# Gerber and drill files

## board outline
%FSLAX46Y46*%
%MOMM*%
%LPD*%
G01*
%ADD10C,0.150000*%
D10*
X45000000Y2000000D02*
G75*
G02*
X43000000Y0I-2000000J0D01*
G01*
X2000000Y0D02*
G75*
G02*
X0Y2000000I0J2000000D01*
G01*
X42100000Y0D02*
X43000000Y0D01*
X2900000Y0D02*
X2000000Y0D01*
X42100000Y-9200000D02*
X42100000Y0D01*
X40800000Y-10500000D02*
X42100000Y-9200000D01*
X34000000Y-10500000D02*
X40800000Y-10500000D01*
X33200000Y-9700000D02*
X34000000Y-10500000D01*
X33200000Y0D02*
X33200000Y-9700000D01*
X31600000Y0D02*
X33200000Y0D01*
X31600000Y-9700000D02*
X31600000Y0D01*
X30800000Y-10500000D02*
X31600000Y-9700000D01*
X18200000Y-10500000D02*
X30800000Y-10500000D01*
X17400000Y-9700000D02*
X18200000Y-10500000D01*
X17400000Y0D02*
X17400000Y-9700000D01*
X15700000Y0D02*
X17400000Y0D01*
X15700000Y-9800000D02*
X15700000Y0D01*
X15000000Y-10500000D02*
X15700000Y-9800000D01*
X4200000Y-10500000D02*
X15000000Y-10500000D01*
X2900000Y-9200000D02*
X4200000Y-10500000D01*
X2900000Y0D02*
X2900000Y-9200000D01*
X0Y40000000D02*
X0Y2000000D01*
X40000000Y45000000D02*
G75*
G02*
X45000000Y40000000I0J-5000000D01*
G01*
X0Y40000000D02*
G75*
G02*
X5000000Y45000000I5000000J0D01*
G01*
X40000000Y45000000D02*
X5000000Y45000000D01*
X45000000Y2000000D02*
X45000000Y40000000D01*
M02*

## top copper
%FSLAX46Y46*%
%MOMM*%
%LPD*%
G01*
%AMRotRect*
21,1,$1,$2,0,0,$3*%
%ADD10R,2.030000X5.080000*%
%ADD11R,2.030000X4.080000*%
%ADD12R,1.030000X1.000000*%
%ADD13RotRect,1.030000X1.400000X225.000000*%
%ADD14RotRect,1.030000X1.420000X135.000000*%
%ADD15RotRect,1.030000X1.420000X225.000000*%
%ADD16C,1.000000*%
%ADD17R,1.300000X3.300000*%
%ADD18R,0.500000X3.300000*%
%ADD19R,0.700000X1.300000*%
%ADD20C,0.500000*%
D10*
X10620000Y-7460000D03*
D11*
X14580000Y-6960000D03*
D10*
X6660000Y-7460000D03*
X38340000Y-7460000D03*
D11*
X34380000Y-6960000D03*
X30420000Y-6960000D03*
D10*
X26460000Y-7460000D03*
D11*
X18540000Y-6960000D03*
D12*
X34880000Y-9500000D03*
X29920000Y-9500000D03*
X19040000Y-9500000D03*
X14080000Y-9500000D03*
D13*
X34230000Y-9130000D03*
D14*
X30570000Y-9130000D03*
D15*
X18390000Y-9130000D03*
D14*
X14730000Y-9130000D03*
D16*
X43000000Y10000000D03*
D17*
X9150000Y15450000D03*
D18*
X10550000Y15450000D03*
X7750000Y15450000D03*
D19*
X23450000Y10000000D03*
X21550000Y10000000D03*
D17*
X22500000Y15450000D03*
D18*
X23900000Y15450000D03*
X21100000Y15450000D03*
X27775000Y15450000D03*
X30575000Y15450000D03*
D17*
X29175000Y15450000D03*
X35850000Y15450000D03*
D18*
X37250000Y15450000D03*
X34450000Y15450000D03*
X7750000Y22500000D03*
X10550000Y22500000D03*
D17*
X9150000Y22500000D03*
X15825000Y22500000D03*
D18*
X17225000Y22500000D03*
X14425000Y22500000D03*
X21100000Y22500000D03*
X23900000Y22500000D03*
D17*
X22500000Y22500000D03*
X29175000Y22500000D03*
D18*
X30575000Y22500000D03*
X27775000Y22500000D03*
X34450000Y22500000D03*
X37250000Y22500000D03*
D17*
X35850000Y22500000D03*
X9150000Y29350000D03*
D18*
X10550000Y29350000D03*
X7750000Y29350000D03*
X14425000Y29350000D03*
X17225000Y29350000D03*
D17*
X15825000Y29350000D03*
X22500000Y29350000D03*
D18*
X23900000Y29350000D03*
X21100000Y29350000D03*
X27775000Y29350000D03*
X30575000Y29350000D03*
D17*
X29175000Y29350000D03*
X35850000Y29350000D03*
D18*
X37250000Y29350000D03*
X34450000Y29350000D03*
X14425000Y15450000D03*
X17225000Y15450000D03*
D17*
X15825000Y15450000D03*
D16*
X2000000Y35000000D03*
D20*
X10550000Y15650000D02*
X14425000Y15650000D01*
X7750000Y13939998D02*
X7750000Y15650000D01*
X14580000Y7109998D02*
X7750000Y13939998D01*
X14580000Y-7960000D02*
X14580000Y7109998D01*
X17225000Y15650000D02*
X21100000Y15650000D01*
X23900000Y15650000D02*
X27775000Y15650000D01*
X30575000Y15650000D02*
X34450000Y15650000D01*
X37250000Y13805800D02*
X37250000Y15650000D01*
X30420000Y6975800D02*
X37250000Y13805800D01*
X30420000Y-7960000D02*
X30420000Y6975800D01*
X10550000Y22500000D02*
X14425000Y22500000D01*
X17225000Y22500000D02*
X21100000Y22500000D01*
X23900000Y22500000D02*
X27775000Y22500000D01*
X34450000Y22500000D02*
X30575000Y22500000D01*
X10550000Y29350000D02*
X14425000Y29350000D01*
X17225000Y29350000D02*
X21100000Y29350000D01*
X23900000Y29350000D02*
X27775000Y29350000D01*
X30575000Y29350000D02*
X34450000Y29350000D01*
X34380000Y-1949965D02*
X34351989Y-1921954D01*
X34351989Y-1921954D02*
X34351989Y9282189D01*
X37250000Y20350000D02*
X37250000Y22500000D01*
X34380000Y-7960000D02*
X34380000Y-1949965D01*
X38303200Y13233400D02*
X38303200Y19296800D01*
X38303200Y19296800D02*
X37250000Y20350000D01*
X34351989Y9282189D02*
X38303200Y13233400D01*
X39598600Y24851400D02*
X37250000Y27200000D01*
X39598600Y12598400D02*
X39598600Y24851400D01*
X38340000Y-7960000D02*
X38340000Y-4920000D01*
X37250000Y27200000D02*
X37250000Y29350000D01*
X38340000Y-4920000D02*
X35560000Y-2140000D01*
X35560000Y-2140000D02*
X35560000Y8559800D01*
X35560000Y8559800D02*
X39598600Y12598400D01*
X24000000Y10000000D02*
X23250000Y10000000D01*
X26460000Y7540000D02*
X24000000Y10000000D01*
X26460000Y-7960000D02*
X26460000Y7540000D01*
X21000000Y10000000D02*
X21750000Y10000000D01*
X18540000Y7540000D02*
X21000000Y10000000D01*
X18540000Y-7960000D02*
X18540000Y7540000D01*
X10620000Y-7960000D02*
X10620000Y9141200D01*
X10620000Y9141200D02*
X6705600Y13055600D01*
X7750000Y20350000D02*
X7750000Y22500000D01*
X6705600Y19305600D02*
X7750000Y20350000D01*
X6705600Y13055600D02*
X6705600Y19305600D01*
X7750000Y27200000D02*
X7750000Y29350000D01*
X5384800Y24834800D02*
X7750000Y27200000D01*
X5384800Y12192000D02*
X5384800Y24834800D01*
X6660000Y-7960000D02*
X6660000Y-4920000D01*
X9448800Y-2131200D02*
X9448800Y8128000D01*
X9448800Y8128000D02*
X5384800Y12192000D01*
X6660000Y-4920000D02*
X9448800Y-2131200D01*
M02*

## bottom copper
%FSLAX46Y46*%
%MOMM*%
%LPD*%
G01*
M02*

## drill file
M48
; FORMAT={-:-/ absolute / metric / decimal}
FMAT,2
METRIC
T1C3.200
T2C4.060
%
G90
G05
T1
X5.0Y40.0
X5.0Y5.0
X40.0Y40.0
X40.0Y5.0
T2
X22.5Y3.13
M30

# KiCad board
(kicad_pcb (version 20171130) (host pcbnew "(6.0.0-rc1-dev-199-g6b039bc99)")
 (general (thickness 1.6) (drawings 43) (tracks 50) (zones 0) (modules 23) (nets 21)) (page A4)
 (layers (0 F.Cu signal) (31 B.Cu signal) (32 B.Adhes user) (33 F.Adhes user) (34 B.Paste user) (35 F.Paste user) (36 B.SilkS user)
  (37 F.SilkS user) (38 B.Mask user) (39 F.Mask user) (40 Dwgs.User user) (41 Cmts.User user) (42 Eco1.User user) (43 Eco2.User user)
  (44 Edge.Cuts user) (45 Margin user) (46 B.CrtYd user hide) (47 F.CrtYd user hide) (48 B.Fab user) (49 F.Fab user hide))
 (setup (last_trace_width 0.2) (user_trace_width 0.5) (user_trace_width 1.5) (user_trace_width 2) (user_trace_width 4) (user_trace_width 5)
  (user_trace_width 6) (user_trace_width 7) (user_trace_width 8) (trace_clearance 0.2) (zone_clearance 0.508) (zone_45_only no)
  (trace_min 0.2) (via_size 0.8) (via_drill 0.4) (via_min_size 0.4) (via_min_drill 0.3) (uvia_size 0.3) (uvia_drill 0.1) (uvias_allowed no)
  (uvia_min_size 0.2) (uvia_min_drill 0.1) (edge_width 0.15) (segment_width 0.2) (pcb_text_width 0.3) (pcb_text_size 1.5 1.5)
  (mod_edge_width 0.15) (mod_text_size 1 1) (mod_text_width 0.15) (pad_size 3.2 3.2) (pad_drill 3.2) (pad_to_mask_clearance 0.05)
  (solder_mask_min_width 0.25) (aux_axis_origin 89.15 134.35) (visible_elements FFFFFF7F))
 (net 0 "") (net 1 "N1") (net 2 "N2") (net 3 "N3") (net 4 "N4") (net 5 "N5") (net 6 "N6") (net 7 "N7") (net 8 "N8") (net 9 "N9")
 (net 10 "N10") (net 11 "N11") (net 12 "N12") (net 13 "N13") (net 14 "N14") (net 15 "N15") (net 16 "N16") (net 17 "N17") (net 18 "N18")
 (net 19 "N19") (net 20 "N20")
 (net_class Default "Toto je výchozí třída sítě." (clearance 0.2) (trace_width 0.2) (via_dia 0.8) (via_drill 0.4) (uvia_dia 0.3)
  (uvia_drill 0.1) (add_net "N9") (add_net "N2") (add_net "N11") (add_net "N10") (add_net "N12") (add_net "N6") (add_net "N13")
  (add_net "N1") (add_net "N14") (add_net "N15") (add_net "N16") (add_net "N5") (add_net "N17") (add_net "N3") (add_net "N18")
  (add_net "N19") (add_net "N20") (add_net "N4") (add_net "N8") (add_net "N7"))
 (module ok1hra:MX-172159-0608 (layer F.Cu) (at 22.5 10.5 180)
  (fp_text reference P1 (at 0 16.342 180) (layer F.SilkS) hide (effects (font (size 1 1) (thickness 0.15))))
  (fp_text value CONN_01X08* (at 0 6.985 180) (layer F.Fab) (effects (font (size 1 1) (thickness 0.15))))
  (pad 2 smd rect (at 11.88 3.04 180) (size 2.03 5.08) (layers F.Cu F.Mask) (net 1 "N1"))
  (pad 3 smd rect (at 7.92 3.54 180) (size 2.03 4.08) (layers F.Cu F.Mask) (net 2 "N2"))
  (pad 1 smd rect (at 15.84 3.04 180) (size 2.03 5.08) (layers F.Cu F.Mask) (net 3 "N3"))
  (pad 8 smd rect (at -15.84 3.04 180) (size 2.03 5.08) (layers F.Cu F.Mask) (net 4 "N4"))
  (pad 7 smd rect (at -11.88 3.54 180) (size 2.03 4.08) (layers F.Cu F.Mask) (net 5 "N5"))
  (pad 6 smd rect (at -7.92 3.54 180) (size 2.03 4.08) (layers F.Cu F.Mask) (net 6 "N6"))
  (pad 5 smd rect (at -3.96 3.04 180) (size 2.03 5.08) (layers F.Cu F.Mask) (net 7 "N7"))
  (pad 4 smd rect (at 3.96 3.54 180) (size 2.03 4.08) (layers F.Cu F.Mask) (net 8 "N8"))
  (pad "" np_thru_hole circle (at 0 13.63 180) (size 4.06 4.06) (drill 4.06) (layers *.Cu *.Mask))
  (pad 7 smd rect (at -12.38 1 180) (size 1.03 1) (layers F.Cu F.Mask) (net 5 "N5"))
  (pad 6 smd rect (at -7.42 1 180) (size 1.03 1) (layers F.Cu F.Mask) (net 6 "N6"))
  (pad 4 smd rect (at 3.46 1 180) (size 1.03 1) (layers F.Cu F.Mask) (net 8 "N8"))
  (pad 3 smd rect (at 8.42 1 180) (size 1.03 1) (layers F.Cu F.Mask) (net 2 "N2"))
  (pad 7 smd rect (at -11.73 1.37 225) (size 1.03 1.4) (layers F.Cu F.Mask) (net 5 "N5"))
  (pad 6 smd rect (at -8.07 1.37 135) (size 1.03 1.42) (layers F.Cu F.Mask) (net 6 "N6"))
  (pad 4 smd rect (at 4.11 1.37 225) (size 1.03 1.42) (layers F.Cu F.Mask) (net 8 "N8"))
  (pad 3 smd rect (at 7.77 1.37 135) (size 1.03 1.42) (layers F.Cu F.Mask) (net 2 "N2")))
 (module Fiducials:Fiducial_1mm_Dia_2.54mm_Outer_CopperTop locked (layer F.Cu) (at 43 -10)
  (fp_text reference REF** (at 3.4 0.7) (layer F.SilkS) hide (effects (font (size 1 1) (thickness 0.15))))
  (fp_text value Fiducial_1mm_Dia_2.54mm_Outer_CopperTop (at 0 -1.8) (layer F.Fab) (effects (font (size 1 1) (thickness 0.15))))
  (pad ~ smd circle (at 0 0) (size 1 1) (layers F.Cu F.Mask) (solder_mask_margin 0.77) (clearance 0.77)))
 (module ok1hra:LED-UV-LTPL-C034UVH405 (layer F.Cu) (at 9.15 -15.45 180)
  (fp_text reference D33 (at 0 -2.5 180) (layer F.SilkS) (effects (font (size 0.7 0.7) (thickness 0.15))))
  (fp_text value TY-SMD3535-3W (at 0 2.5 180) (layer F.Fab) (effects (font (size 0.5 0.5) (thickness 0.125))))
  (pad 3 smd rect (at 0 0 180) (size 1.3 3.3) (layers F.Cu F.Paste F.Mask))
  (pad 1 smd rect (at -1.4 0 180) (size 0.5 3.3) (layers F.Cu F.Paste F.Mask) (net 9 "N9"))
  (pad 2 smd rect (at 1.4 0 180) (size 0.5 3.3) (layers F.Cu F.Paste F.Mask) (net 2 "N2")))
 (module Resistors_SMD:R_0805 (layer F.Cu) (at 22.5 -10 180)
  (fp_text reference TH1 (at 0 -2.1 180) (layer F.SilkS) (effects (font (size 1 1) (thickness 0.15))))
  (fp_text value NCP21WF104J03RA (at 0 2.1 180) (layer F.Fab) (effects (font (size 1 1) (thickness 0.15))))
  (pad 1 smd rect (at -0.95 0 180) (size 0.7 1.3) (layers F.Cu F.Paste F.Mask) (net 7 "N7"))
  (pad 2 smd rect (at 0.95 0 180) (size 0.7 1.3) (layers F.Cu F.Paste F.Mask) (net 8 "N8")))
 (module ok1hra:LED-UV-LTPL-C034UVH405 (layer F.Cu) (at 22.5 -15.45 180)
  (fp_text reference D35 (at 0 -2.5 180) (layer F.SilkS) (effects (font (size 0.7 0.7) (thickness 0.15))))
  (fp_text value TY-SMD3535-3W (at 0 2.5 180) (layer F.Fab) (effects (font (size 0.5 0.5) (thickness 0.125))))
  (pad 3 smd rect (at 0 0 180) (size 1.3 3.3) (layers F.Cu F.Paste F.Mask))
  (pad 1 smd rect (at -1.4 0 180) (size 0.5 3.3) (layers F.Cu F.Paste F.Mask) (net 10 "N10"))
  (pad 2 smd rect (at 1.4 0 180) (size 0.5 3.3) (layers F.Cu F.Paste F.Mask) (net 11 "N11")))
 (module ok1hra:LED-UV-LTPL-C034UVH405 (layer F.Cu) (at 29.175 -15.45 180)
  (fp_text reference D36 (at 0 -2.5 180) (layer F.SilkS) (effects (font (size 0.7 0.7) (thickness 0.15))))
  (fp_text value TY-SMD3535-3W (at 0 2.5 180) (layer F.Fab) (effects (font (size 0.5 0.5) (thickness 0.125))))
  (pad 2 smd rect (at 1.4 0 180) (size 0.5 3.3) (layers F.Cu F.Paste F.Mask) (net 10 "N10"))
  (pad 1 smd rect (at -1.4 0 180) (size 0.5 3.3) (layers F.Cu F.Paste F.Mask) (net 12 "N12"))
  (pad 3 smd rect (at 0 0 180) (size 1.3 3.3) (layers F.Cu F.Paste F.Mask)))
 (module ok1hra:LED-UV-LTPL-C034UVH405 (layer F.Cu) (at 35.85 -15.45 180)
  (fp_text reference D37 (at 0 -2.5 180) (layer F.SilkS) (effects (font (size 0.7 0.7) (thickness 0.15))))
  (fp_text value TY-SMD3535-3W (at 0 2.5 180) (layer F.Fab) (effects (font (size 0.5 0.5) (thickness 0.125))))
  (pad 3 smd rect (at 0 0 180) (size 1.3 3.3) (layers F.Cu F.Paste F.Mask))
  (pad 1 smd rect (at -1.4 0 180) (size 0.5 3.3) (layers F.Cu F.Paste F.Mask) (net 6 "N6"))
  (pad 2 smd rect (at 1.4 0 180) (size 0.5 3.3) (layers F.Cu F.Paste F.Mask) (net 12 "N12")))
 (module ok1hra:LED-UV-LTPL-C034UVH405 (layer F.Cu) (at 9.15 -22.5 180)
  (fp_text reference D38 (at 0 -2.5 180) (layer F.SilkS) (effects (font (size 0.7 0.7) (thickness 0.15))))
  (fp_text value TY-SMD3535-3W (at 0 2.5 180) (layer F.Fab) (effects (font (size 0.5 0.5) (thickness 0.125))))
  (pad 2 smd rect (at 1.4 0 180) (size 0.5 3.3) (layers F.Cu F.Paste F.Mask) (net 1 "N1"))
  (pad 1 smd rect (at -1.4 0 180) (size 0.5 3.3) (layers F.Cu F.Paste F.Mask) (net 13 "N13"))
  (pad 3 smd rect (at 0 0 180) (size 1.3 3.3) (layers F.Cu F.Paste F.Mask)))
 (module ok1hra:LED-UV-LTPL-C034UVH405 (layer F.Cu) (at 15.825 -22.5 180)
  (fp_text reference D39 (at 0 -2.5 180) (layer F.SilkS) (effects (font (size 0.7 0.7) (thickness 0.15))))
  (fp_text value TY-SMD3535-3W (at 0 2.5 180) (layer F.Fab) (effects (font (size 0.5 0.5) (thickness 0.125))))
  (pad 3 smd rect (at 0 0 180) (size 1.3 3.3) (layers F.Cu F.Paste F.Mask))
  (pad 1 smd rect (at -1.4 0 180) (size 0.5 3.3) (layers F.Cu F.Paste F.Mask) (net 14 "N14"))
  (pad 2 smd rect (at 1.4 0 180) (size 0.5 3.3) (layers F.Cu F.Paste F.Mask) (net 13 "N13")))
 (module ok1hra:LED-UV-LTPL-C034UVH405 (layer F.Cu) (at 22.5 -22.5 180)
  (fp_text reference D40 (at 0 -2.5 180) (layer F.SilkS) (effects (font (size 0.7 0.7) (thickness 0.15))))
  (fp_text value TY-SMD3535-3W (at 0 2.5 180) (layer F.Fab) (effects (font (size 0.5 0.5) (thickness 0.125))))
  (pad 2 smd rect (at 1.4 0 180) (size 0.5 3.3) (layers F.Cu F.Paste F.Mask) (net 14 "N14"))
  (pad 1 smd rect (at -1.4 0 180) (size 0.5 3.3) (layers F.Cu F.Paste F.Mask) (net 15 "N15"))
  (pad 3 smd rect (at 0 0 180) (size 1.3 3.3) (layers F.Cu F.Paste F.Mask)))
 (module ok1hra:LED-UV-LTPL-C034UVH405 (layer F.Cu) (at 29.175 -22.5 180)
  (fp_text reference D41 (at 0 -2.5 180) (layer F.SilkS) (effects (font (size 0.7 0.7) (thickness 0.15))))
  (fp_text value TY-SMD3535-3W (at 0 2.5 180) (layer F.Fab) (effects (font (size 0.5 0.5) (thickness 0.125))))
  (pad 3 smd rect (at 0 0 180) (size 1.3 3.3) (layers F.Cu F.Paste F.Mask))
  (pad 1 smd rect (at -1.4 0 180) (size 0.5 3.3) (layers F.Cu F.Paste F.Mask) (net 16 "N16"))
  (pad 2 smd rect (at 1.4 0 180) (size 0.5 3.3) (layers F.Cu F.Paste F.Mask) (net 15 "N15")))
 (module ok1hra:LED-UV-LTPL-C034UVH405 (layer F.Cu) (at 35.85 -22.5 180)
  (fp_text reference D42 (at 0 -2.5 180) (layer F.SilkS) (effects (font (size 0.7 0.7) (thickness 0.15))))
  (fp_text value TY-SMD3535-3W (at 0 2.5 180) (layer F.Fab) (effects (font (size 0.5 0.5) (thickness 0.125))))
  (pad 2 smd rect (at 1.4 0 180) (size 0.5 3.3) (layers F.Cu F.Paste F.Mask) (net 16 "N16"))
  (pad 1 smd rect (at -1.4 0 180) (size 0.5 3.3) (layers F.Cu F.Paste F.Mask) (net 5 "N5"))
  (pad 3 smd rect (at 0 0 180) (size 1.3 3.3) (layers F.Cu F.Paste F.Mask)))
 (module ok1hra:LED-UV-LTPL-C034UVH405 (layer F.Cu) (at 9.15 -29.35 180)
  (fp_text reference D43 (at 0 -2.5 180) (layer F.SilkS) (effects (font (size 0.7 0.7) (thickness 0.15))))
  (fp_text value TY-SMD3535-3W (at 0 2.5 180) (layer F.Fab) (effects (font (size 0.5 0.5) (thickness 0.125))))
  (pad 3 smd rect (at 0 0 180) (size 1.3 3.3) (layers F.Cu F.Paste F.Mask))
  (pad 1 smd rect (at -1.4 0 180) (size 0.5 3.3) (layers F.Cu F.Paste F.Mask) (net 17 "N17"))
  (pad 2 smd rect (at 1.4 0 180) (size 0.5 3.3) (layers F.Cu F.Paste F.Mask) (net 3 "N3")))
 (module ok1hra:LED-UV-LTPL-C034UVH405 (layer F.Cu) (at 15.825 -29.35 180)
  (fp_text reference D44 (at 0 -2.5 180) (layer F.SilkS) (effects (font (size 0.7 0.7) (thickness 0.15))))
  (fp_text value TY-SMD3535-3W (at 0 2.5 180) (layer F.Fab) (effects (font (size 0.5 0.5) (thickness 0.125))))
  (pad 2 smd rect (at 1.4 0 180) (size 0.5 3.3) (layers F.Cu F.Paste F.Mask) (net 17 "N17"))
  (pad 1 smd rect (at -1.4 0 180) (size 0.5 3.3) (layers F.Cu F.Paste F.Mask) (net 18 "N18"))
  (pad 3 smd rect (at 0 0 180) (size 1.3 3.3) (layers F.Cu F.Paste F.Mask)))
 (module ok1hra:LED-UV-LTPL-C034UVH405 (layer F.Cu) (at 22.5 -29.35 180)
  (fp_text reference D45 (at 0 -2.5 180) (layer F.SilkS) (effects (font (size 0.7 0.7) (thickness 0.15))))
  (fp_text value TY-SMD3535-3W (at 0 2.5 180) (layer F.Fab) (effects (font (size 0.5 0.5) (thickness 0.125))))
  (pad 3 smd rect (at 0 0 180) (size 1.3 3.3) (layers F.Cu F.Paste F.Mask))
  (pad 1 smd rect (at -1.4 0 180) (size 0.5 3.3) (layers F.Cu F.Paste F.Mask) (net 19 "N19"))
  (pad 2 smd rect (at 1.4 0 180) (size 0.5 3.3) (layers F.Cu F.Paste F.Mask) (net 18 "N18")))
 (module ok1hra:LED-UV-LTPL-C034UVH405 (layer F.Cu) (at 29.175 -29.35 180)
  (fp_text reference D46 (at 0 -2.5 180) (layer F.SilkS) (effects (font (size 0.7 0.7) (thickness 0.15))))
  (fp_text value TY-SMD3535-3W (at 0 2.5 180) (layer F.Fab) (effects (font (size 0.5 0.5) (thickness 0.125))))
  (pad 2 smd rect (at 1.4 0 180) (size 0.5 3.3) (layers F.Cu F.Paste F.Mask) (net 19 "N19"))
  (pad 1 smd rect (at -1.4 0 180) (size 0.5 3.3) (layers F.Cu F.Paste F.Mask) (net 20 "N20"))
  (pad 3 smd rect (at 0 0 180) (size 1.3 3.3) (layers F.Cu F.Paste F.Mask)))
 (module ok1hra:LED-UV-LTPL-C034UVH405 (layer F.Cu) (at 35.85 -29.35 180)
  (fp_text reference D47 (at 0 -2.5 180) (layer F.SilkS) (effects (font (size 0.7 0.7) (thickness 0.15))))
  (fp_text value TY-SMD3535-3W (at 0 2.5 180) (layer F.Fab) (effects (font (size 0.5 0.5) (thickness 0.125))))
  (pad 3 smd rect (at 0 0 180) (size 1.3 3.3) (layers F.Cu F.Paste F.Mask))
  (pad 1 smd rect (at -1.4 0 180) (size 0.5 3.3) (layers F.Cu F.Paste F.Mask) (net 4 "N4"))
  (pad 2 smd rect (at 1.4 0 180) (size 0.5 3.3) (layers F.Cu F.Paste F.Mask) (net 20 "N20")))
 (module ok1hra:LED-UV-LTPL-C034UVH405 (layer F.Cu) (at 15.825 -15.45 180)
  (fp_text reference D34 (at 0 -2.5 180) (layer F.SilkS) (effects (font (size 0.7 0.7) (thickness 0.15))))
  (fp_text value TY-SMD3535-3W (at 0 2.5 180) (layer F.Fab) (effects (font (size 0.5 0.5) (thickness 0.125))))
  (pad 2 smd rect (at 1.4 0 180) (size 0.5 3.3) (layers F.Cu F.Paste F.Mask) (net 9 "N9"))
  (pad 1 smd rect (at -1.4 0 180) (size 0.5 3.3) (layers F.Cu F.Paste F.Mask) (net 11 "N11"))
  (pad 3 smd rect (at 0 0 180) (size 1.3 3.3) (layers F.Cu F.Paste F.Mask)))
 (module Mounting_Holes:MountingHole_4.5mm (layer F.Cu) (at 40 -40)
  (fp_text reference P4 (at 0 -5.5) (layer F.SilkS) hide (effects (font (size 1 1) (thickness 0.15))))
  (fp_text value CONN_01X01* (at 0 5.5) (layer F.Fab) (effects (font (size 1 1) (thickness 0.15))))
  (pad "" np_thru_hole circle (at 0 0) (size 3.2 3.2) (drill 3.2) (layers *.Cu *.Mask)))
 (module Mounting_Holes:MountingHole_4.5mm (layer F.Cu) (at 40 -5)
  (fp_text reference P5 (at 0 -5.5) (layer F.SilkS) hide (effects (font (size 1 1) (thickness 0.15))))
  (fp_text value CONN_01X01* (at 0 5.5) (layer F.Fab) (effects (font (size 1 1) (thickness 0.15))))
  (pad "" np_thru_hole circle (at 0 0) (size 3.2 3.2) (drill 3.2) (layers *.Cu *.Mask)))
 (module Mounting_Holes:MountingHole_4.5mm (layer F.Cu) (at 5 -5)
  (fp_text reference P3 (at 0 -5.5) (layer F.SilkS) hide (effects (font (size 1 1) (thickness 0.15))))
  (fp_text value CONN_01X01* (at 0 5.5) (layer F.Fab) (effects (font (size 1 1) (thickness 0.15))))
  (pad "" np_thru_hole circle (at 0 0) (size 3.2 3.2) (drill 3.2) (layers *.Cu *.Mask)))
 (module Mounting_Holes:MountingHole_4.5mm (layer F.Cu) (at 5 -40)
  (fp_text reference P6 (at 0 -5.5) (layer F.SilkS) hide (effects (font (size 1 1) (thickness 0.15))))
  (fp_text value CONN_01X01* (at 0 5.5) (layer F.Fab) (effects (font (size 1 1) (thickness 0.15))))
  (pad "" np_thru_hole circle (at 0 0) (size 3.2 3.2) (drill 3.2) (layers *.Cu *.Mask)))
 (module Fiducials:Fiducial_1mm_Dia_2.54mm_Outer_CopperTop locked (layer F.Cu) (at 2 -35)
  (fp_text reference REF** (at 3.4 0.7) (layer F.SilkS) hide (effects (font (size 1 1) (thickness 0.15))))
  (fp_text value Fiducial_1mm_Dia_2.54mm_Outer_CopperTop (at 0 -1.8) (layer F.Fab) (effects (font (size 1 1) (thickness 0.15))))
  (pad ~ smd circle (at 0 0) (size 1 1) (layers F.Cu F.Mask) (solder_mask_margin 0.77) (clearance 0.77)))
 (gr_arc (start 43 -2) (end 43 0) (angle -90) (layer Edge.Cuts) (width 0.15))
 (gr_arc (start 2 -2) (end 0 -2) (angle -90) (layer Edge.Cuts) (width 0.15))
 (gr_line (start 42.1 0) (end 43 0) (layer Edge.Cuts) (width 0.15))
 (gr_line (start 2.9 0) (end 2 0) (layer Edge.Cuts) (width 0.15))
 (gr_line (start 42.1 9.2) (end 42.1 0) (layer Edge.Cuts) (width 0.15))
 (gr_line (start 40.8 10.5) (end 42.1 9.2) (layer Edge.Cuts) (width 0.15))
 (gr_line (start 34 10.5) (end 40.8 10.5) (layer Edge.Cuts) (width 0.15))
 (gr_line (start 33.2 9.7) (end 34 10.5) (layer Edge.Cuts) (width 0.15))
 (gr_line (start 33.2 0) (end 33.2 9.7) (layer Edge.Cuts) (width 0.15))
 (gr_line (start 31.6 0) (end 33.2 0) (layer Edge.Cuts) (width 0.15))
 (gr_line (start 31.6 9.7) (end 31.6 0) (layer Edge.Cuts) (width 0.15))
 (gr_line (start 30.8 10.5) (end 31.6 9.7) (layer Edge.Cuts) (width 0.15))
 (gr_line (start 18.2 10.5) (end 30.8 10.5) (layer Edge.Cuts) (width 0.15))
 (gr_line (start 17.4 9.7) (end 18.2 10.5) (layer Edge.Cuts) (width 0.15))
 (gr_line (start 17.4 0) (end 17.4 9.7) (layer Edge.Cuts) (width 0.15))
 (gr_line (start 15.7 0) (end 17.4 0) (layer Edge.Cuts) (width 0.15))
 (gr_line (start 15.7 9.8) (end 15.7 0) (layer Edge.Cuts) (width 0.15))
 (gr_line (start 15 10.5) (end 15.7 9.8) (layer Edge.Cuts) (width 0.15))
 (gr_line (start 4.2 10.5) (end 15 10.5) (layer Edge.Cuts) (width 0.15))
 (gr_line (start 2.9 9.2) (end 4.2 10.5) (layer Edge.Cuts) (width 0.15))
 (gr_line (start 2.9 0) (end 2.9 9.2) (layer Edge.Cuts) (width 0.15))
 (gr_line (start 0 -40) (end 0 -2) (layer Edge.Cuts) (width 0.15))
 (gr_arc (start 40 -40) (end 45 -40) (angle -90) (layer Edge.Cuts) (width 0.15))
 (gr_arc (start 5 -40) (end 5 -45) (angle -90) (layer Edge.Cuts) (width 0.15))
 (gr_line (start 40 -45) (end 5 -45) (layer Edge.Cuts) (width 0.15))
 (gr_line (start 45 -2) (end 45 -40) (layer Edge.Cuts) (width 0.15))
 (segment (start 10.55 -15.65) (end 14.425 -15.65) (width 0.5) (layer F.Cu) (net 9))
 (segment (start 7.75 -13.939998) (end 7.75 -15.65) (width 0.5) (layer F.Cu) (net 2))
 (segment (start 14.58 -7.109998) (end 7.75 -13.939998) (width 0.5) (layer F.Cu) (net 2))
 (segment (start 14.58 7.96) (end 14.58 -7.109998) (width 0.5) (layer F.Cu) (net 2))
 (segment (start 17.225 -15.65) (end 21.1 -15.65) (width 0.5) (layer F.Cu) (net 11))
 (segment (start 23.9 -15.65) (end 27.775 -15.65) (width 0.5) (layer F.Cu) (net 10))
 (segment (start 30.575 -15.65) (end 34.45 -15.65) (width 0.5) (layer F.Cu) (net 12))
 (segment (start 37.25 -13.8058) (end 37.25 -15.65) (width 0.5) (layer F.Cu) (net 6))
 (segment (start 30.42 -6.9758) (end 37.25 -13.8058) (width 0.5) (layer F.Cu) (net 6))
 (segment (start 30.42 7.96) (end 30.42 -6.9758) (width 0.5) (layer F.Cu) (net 6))
 (segment (start 10.55 -22.5) (end 14.425 -22.5) (width 0.5) (layer F.Cu) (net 13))
 (segment (start 17.225 -22.5) (end 21.1 -22.5) (width 0.5) (layer F.Cu) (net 14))
 (segment (start 23.9 -22.5) (end 27.775 -22.5) (width 0.5) (layer F.Cu) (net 15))
 (segment (start 34.45 -22.5) (end 30.575 -22.5) (width 0.5) (layer F.Cu) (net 16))
 (segment (start 10.55 -29.35) (end 14.425 -29.35) (width 0.5) (layer F.Cu) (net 17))
 (segment (start 17.225 -29.35) (end 21.1 -29.35) (width 0.5) (layer F.Cu) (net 18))
 (segment (start 23.9 -29.35) (end 27.775 -29.35) (width 0.5) (layer F.Cu) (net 19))
 (segment (start 30.575 -29.35) (end 34.45 -29.35) (width 0.5) (layer F.Cu) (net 20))
 (segment (start 34.38 1.949965) (end 34.351989 1.921954) (width 0.5) (layer F.Cu) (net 5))
 (segment (start 34.351989 1.921954) (end 34.351989 -9.282189) (width 0.5) (layer F.Cu) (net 5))
 (segment (start 37.25 -20.35) (end 37.25 -22.5) (width 0.5) (layer F.Cu) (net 5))
 (segment (start 34.38 7.96) (end 34.38 1.949965) (width 0.5) (layer F.Cu) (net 5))
 (segment (start 38.3032 -13.2334) (end 38.3032 -19.2968) (width 0.5) (layer F.Cu) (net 5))
 (segment (start 38.3032 -19.2968) (end 37.25 -20.35) (width 0.5) (layer F.Cu) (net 5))
 (segment (start 34.351989 -9.282189) (end 38.3032 -13.2334) (width 0.5) (layer F.Cu) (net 5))
 (segment (start 39.5986 -24.8514) (end 37.25 -27.2) (width 0.5) (layer F.Cu) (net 4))
 (segment (start 39.5986 -12.5984) (end 39.5986 -24.8514) (width 0.5) (layer F.Cu) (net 4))
 (segment (start 38.34 7.96) (end 38.34 4.92) (width 0.5) (layer F.Cu) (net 4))
 (segment (start 37.25 -27.2) (end 37.25 -29.35) (width 0.5) (layer F.Cu) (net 4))
 (segment (start 38.34 4.92) (end 35.56 2.14) (width 0.5) (layer F.Cu) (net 4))
 (segment (start 35.56 2.14) (end 35.56 -8.5598) (width 0.5) (layer F.Cu) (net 4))
 (segment (start 35.56 -8.5598) (end 39.5986 -12.5984) (width 0.5) (layer F.Cu) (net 4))
 (segment (start 24 -10) (end 23.25 -10) (width 0.5) (layer F.Cu) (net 7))
 (segment (start 26.46 -7.54) (end 24 -10) (width 0.5) (layer F.Cu) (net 7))
 (segment (start 26.46 7.96) (end 26.46 -7.54) (width 0.5) (layer F.Cu) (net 7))
 (segment (start 21 -10) (end 21.75 -10) (width 0.5) (layer F.Cu) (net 8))
 (segment (start 18.54 -7.54) (end 21 -10) (width 0.5) (layer F.Cu) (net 8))
 (segment (start 18.54 7.96) (end 18.54 -7.54) (width 0.5) (layer F.Cu) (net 8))
 (segment (start 10.62 7.96) (end 10.62 -9.1412) (width 0.5) (layer F.Cu) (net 1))
 (segment (start 10.62 -9.1412) (end 6.7056 -13.0556) (width 0.5) (layer F.Cu) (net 1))
 (segment (start 7.75 -20.35) (end 7.75 -22.5) (width 0.5) (layer F.Cu) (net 1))
 (segment (start 6.7056 -19.3056) (end 7.75 -20.35) (width 0.5) (layer F.Cu) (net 1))
 (segment (start 6.7056 -13.0556) (end 6.7056 -19.3056) (width 0.5) (layer F.Cu) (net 1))
 (segment (start 7.75 -27.2) (end 7.75 -29.35) (width 0.5) (layer F.Cu) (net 3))
 (segment (start 5.3848 -24.8348) (end 7.75 -27.2) (width 0.5) (layer F.Cu) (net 3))
 (segment (start 5.3848 -12.192) (end 5.3848 -24.8348) (width 0.5) (layer F.Cu) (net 3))
 (segment (start 6.66 7.96) (end 6.66 4.92) (width 0.5) (layer F.Cu) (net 3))
 (segment (start 9.4488 2.1312) (end 9.4488 -8.128) (width 0.5) (layer F.Cu) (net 3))
 (segment (start 9.4488 -8.128) (end 5.3848 -12.192) (width 0.5) (layer F.Cu) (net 3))
 (segment (start 6.66 4.92) (end 9.4488 2.1312) (width 0.5) (layer F.Cu) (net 3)))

